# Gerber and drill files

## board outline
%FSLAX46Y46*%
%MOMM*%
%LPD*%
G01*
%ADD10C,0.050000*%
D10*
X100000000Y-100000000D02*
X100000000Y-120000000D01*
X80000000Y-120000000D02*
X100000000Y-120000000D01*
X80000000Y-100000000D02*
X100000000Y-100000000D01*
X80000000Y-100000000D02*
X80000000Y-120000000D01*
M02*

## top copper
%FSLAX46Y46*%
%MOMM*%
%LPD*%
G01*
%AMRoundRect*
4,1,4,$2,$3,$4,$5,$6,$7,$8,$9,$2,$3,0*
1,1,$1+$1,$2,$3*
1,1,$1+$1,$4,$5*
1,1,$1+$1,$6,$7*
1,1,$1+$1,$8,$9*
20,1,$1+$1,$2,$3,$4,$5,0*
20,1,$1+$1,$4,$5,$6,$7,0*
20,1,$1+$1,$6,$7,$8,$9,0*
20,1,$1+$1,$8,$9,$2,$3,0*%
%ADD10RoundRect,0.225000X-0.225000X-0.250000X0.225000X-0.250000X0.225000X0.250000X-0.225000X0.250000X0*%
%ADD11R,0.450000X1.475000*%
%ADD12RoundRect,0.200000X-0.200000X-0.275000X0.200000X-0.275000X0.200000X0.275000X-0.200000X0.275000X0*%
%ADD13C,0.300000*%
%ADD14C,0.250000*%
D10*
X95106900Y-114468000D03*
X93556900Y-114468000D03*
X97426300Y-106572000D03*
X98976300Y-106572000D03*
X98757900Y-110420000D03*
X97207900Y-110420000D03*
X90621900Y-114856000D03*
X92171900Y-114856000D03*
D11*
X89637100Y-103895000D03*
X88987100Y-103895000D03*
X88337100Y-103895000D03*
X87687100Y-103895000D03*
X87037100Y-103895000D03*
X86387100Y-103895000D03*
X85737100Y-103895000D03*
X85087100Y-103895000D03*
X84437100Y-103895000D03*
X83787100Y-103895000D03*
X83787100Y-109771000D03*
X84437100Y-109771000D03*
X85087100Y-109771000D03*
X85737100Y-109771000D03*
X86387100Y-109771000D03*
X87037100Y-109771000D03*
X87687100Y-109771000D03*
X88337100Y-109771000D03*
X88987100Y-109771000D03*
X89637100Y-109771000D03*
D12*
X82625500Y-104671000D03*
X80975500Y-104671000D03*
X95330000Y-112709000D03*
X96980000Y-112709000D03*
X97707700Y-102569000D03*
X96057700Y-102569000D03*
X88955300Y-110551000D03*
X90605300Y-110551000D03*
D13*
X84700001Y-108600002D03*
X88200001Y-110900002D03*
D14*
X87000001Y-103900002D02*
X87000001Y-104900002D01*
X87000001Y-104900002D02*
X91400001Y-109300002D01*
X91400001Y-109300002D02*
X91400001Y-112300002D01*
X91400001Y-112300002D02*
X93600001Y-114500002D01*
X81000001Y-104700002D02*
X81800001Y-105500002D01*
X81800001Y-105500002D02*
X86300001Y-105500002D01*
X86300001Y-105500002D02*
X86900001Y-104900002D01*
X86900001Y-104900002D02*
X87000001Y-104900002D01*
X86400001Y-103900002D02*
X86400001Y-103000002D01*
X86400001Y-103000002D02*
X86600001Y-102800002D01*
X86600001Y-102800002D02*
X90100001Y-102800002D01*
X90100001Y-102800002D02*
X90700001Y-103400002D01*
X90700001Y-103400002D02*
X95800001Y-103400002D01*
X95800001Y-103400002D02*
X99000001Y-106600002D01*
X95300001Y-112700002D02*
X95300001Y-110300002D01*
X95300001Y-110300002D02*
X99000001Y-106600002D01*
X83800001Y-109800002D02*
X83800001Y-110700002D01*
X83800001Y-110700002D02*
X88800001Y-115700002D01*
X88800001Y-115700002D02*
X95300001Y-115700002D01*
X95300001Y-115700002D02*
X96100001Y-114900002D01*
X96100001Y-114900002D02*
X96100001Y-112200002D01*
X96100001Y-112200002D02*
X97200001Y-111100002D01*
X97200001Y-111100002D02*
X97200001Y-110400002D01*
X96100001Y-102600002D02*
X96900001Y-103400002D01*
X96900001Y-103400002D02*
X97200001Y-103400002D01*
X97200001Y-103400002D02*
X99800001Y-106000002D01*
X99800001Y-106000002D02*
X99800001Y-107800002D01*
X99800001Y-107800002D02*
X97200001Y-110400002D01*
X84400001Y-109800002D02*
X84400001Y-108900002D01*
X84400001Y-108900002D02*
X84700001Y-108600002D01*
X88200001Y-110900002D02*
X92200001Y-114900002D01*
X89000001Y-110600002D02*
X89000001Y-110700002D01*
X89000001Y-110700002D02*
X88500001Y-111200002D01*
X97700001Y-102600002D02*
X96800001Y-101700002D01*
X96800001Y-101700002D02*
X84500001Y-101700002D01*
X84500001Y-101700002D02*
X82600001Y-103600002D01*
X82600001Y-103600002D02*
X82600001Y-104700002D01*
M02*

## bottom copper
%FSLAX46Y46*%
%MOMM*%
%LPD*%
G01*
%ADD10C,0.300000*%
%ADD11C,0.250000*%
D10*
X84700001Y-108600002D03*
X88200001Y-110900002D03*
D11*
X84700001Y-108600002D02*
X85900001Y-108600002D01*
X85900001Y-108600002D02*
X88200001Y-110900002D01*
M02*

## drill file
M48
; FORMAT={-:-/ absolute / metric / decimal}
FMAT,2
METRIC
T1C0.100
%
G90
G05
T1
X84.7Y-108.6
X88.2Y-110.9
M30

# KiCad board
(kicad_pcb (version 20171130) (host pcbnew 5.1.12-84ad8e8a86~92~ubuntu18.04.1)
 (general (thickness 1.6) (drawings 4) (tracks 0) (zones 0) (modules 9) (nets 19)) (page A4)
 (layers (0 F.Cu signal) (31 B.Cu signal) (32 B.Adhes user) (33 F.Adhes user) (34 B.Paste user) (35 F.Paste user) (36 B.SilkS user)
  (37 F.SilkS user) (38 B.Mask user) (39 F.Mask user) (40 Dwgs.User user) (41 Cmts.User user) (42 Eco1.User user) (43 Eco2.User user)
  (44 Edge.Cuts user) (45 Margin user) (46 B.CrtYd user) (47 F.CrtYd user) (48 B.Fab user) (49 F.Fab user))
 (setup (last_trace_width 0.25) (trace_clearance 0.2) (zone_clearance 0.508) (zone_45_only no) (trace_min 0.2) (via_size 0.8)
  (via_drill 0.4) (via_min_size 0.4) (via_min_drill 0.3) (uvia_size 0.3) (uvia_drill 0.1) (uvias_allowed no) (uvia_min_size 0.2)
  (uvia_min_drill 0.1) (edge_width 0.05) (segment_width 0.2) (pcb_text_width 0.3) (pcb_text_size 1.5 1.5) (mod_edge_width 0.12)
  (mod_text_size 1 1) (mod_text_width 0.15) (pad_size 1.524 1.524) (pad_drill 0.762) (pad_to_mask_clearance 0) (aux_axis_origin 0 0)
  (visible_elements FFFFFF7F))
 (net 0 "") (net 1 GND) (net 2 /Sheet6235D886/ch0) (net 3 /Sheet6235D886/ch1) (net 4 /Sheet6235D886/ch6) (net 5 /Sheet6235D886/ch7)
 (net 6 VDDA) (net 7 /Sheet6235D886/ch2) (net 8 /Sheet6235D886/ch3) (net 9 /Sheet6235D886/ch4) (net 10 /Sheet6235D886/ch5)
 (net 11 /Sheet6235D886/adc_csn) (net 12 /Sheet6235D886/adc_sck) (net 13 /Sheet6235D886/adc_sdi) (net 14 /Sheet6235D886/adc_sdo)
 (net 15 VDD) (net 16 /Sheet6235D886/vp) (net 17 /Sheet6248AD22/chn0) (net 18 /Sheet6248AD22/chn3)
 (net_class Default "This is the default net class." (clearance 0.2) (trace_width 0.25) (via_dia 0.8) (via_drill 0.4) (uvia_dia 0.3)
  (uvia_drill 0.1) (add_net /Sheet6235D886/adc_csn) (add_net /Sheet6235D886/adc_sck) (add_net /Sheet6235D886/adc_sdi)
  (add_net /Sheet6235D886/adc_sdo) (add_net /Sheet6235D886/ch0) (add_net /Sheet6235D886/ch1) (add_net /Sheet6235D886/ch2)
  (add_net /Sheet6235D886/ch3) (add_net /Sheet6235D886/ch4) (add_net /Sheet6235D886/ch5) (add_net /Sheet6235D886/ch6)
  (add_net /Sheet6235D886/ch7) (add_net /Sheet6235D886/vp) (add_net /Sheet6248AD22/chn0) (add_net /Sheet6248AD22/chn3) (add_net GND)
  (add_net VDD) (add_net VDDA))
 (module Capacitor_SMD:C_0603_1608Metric (layer F.Cu) (at 94.331900 114.468000)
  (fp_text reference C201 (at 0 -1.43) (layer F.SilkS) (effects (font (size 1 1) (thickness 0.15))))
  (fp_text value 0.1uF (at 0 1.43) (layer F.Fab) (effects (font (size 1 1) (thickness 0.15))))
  (pad 2 smd roundrect (at 0.775 0) (size 0.9 0.95) (layers F.Cu F.Mask F.Paste) (roundrect_rratio 0.25) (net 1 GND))
  (pad 1 smd roundrect (at -0.775 0) (size 0.9 0.95) (layers F.Cu F.Mask F.Paste) (roundrect_rratio 0.25) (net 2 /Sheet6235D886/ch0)))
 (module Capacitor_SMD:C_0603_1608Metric (layer F.Cu) (at 98.201300 106.572000)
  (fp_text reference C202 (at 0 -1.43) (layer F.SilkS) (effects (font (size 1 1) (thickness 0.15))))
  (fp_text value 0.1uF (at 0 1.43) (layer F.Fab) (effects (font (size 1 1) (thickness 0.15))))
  (pad 1 smd roundrect (at -0.775 0) (size 0.9 0.95) (layers F.Cu F.Mask F.Paste) (roundrect_rratio 0.25) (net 1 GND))
  (pad 2 smd roundrect (at 0.775 0) (size 0.9 0.95) (layers F.Cu F.Mask F.Paste) (roundrect_rratio 0.25) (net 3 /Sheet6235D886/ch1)))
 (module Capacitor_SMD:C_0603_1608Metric (layer F.Cu) (at 97.982900 110.420000)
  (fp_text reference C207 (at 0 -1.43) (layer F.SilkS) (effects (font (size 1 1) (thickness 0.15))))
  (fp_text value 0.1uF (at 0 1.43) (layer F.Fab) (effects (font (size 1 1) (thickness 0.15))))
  (pad 2 smd roundrect (at 0.775 0) (size 0.9 0.95) (layers F.Cu F.Mask F.Paste) (roundrect_rratio 0.25) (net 1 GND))
  (pad 1 smd roundrect (at -0.775 0) (size 0.9 0.95) (layers F.Cu F.Mask F.Paste) (roundrect_rratio 0.25) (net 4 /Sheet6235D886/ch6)))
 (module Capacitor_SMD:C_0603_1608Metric (layer F.Cu) (at 91.396900 114.856000)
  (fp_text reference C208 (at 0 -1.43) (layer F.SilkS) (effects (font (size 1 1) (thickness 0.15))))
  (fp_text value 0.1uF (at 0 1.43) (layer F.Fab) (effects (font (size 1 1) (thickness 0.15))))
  (pad 1 smd roundrect (at -0.775 0) (size 0.9 0.95) (layers F.Cu F.Mask F.Paste) (roundrect_rratio 0.25) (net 1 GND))
  (pad 2 smd roundrect (at 0.775 0) (size 0.9 0.95) (layers F.Cu F.Mask F.Paste) (roundrect_rratio 0.25) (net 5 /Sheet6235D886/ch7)))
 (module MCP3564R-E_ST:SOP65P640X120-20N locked (layer F.Cu) (at 86.712100 106.833000 270.000000)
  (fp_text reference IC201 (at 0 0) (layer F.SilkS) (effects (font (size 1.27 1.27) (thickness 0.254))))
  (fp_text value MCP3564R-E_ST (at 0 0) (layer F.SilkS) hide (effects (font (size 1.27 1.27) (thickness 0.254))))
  (pad 1 smd rect (at -2.938 -2.925) (size 0.45 1.475) (layers F.Cu F.Mask F.Paste) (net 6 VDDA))
  (pad 2 smd rect (at -2.938 -2.275) (size 0.45 1.475) (layers F.Cu F.Mask F.Paste) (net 1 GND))
  (pad 3 smd rect (at -2.938 -1.625) (size 0.45 1.475) (layers F.Cu F.Mask F.Paste) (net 1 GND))
  (pad 4 smd rect (at -2.938 -0.975) (size 0.45 1.475) (layers F.Cu F.Mask F.Paste))
  (pad 5 smd rect (at -2.938 -0.325) (size 0.45 1.475) (layers F.Cu F.Mask F.Paste) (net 2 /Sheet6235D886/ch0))
  (pad 6 smd rect (at -2.938 0.325) (size 0.45 1.475) (layers F.Cu F.Mask F.Paste) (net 3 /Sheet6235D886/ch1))
  (pad 7 smd rect (at -2.938 0.975) (size 0.45 1.475) (layers F.Cu F.Mask F.Paste) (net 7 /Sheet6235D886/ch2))
  (pad 8 smd rect (at -2.938 1.625) (size 0.45 1.475) (layers F.Cu F.Mask F.Paste) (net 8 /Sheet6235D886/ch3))
  (pad 9 smd rect (at -2.938 2.275) (size 0.45 1.475) (layers F.Cu F.Mask F.Paste) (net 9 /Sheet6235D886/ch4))
  (pad 10 smd rect (at -2.938 2.925) (size 0.45 1.475) (layers F.Cu F.Mask F.Paste) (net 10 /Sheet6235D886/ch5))
  (pad 11 smd rect (at 2.938 2.925) (size 0.45 1.475) (layers F.Cu F.Mask F.Paste) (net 4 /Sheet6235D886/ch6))
  (pad 12 smd rect (at 2.938 2.275) (size 0.45 1.475) (layers F.Cu F.Mask F.Paste) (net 5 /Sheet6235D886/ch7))
  (pad 13 smd rect (at 2.938 1.625) (size 0.45 1.475) (layers F.Cu F.Mask F.Paste) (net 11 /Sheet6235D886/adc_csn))
  (pad 14 smd rect (at 2.938 0.975) (size 0.45 1.475) (layers F.Cu F.Mask F.Paste) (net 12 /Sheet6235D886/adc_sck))
  (pad 15 smd rect (at 2.938 0.325) (size 0.45 1.475) (layers F.Cu F.Mask F.Paste) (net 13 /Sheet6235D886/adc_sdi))
  (pad 16 smd rect (at 2.938 -0.325) (size 0.45 1.475) (layers F.Cu F.Mask F.Paste) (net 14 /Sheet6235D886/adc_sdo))
  (pad 17 smd rect (at 2.938 -0.975) (size 0.45 1.475) (layers F.Cu F.Mask F.Paste))
  (pad 18 smd rect (at 2.938 -1.625) (size 0.45 1.475) (layers F.Cu F.Mask F.Paste))
  (pad 19 smd rect (at 2.938 -2.275) (size 0.45 1.475) (layers F.Cu F.Mask F.Paste) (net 1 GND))
  (pad 20 smd rect (at 2.938 -2.925) (size 0.45 1.475) (layers F.Cu F.Mask F.Paste) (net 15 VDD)))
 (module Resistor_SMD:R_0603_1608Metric (layer F.Cu) (at 81.800500 104.671000)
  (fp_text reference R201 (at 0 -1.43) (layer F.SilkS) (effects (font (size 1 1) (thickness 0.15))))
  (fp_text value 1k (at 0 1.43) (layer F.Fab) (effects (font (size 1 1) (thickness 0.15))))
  (pad 2 smd roundrect (at 0.825 0) (size 0.8 0.95) (layers F.Cu F.Mask F.Paste) (roundrect_rratio 0.25) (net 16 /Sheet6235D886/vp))
  (pad 1 smd roundrect (at -0.825 0) (size 0.8 0.95) (layers F.Cu F.Mask F.Paste) (roundrect_rratio 0.25) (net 2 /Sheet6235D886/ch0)))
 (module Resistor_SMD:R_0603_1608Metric (layer F.Cu) (at 96.155000 112.709000)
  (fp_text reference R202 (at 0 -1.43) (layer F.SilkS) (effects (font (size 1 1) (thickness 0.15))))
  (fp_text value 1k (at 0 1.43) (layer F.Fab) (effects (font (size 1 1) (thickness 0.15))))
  (pad 1 smd roundrect (at -0.825 0) (size 0.8 0.95) (layers F.Cu F.Mask F.Paste) (roundrect_rratio 0.25) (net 3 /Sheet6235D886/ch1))
  (pad 2 smd roundrect (at 0.825 0) (size 0.8 0.95) (layers F.Cu F.Mask F.Paste) (roundrect_rratio 0.25) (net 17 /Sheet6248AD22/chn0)))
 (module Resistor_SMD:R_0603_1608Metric (layer F.Cu) (at 96.882700 102.569000)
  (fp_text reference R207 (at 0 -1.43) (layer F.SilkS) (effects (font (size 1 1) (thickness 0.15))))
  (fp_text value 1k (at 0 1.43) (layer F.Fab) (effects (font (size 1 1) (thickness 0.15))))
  (pad 2 smd roundrect (at 0.825 0) (size 0.8 0.95) (layers F.Cu F.Mask F.Paste) (roundrect_rratio 0.25) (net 16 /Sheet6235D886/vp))
  (pad 1 smd roundrect (at -0.825 0) (size 0.8 0.95) (layers F.Cu F.Mask F.Paste) (roundrect_rratio 0.25) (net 4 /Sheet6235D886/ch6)))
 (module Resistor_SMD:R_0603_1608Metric (layer F.Cu) (at 89.780300 110.551000)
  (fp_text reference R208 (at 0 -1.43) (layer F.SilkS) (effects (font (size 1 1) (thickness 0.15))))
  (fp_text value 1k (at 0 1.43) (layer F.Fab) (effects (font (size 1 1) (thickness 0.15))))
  (pad 1 smd roundrect (at -0.825 0) (size 0.8 0.95) (layers F.Cu F.Mask F.Paste) (roundrect_rratio 0.25) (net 5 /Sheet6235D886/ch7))
  (pad 2 smd roundrect (at 0.825 0) (size 0.8 0.95) (layers F.Cu F.Mask F.Paste) (roundrect_rratio 0.25) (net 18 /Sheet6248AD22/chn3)))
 (gr_line (start 100 100) (end 100 120) (layer Edge.Cuts) (width 0.05))
 (gr_line (start 80 120) (end 100 120) (layer Edge.Cuts) (width 0.05))
 (gr_line (start 80 100) (end 100 100) (layer Edge.Cuts) (width 0.05))
 (gr_line (start 80 100) (end 80 120) (layer Edge.Cuts) (width 0.05))
 (segment (start 87.000001 103.900002) (end 87.000001 104.900002) (width 0.250000) (layer F.Cu) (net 2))
 (segment (start 87.000001 104.900002) (end 91.400001 109.300002) (width 0.250000) (layer F.Cu) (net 2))
 (segment (start 91.400001 109.300002) (end 91.400001 112.300002) (width 0.250000) (layer F.Cu) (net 2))
 (segment (start 91.400001 112.300002) (end 93.600001 114.500002) (width 0.250000) (layer F.Cu) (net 2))
 (segment (start 81.000001 104.700002) (end 81.800001 105.500002) (width 0.250000) (layer F.Cu) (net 2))
 (segment (start 81.800001 105.500002) (end 86.300001 105.500002) (width 0.250000) (layer F.Cu) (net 2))
 (segment (start 86.300001 105.500002) (end 86.900001 104.900002) (width 0.250000) (layer F.Cu) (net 2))
 (segment (start 86.900001 104.900002) (end 87.000001 104.900002) (width 0.250000) (layer F.Cu) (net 2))
 (segment (start 86.400001 103.900002) (end 86.400001 103.000002) (width 0.250000) (layer F.Cu) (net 3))
 (segment (start 86.400001 103.000002) (end 86.600001 102.800002) (width 0.250000) (layer F.Cu) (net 3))
 (segment (start 86.600001 102.800002) (end 90.100001 102.800002) (width 0.250000) (layer F.Cu) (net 3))
 (segment (start 90.100001 102.800002) (end 90.700001 103.400002) (width 0.250000) (layer F.Cu) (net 3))
 (segment (start 90.700001 103.400002) (end 95.800001 103.400002) (width 0.250000) (layer F.Cu) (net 3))
 (segment (start 95.800001 103.400002) (end 99.000001 106.600002) (width 0.250000) (layer F.Cu) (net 3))
 (segment (start 95.300001 112.700002) (end 95.300001 110.300002) (width 0.250000) (layer F.Cu) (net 3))
 (segment (start 95.300001 110.300002) (end 99.000001 106.600002) (width 0.250000) (layer F.Cu) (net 3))
 (segment (start 83.800001 109.800002) (end 83.800001 110.700002) (width 0.250000) (layer F.Cu) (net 4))
 (segment (start 83.800001 110.700002) (end 88.800001 115.700002) (width 0.250000) (layer F.Cu) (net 4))
 (segment (start 88.800001 115.700002) (end 95.300001 115.700002) (width 0.250000) (layer F.Cu) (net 4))
 (segment (start 95.300001 115.700002) (end 96.100001 114.900002) (width 0.250000) (layer F.Cu) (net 4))
 (segment (start 96.100001 114.900002) (end 96.100001 112.200002) (width 0.250000) (layer F.Cu) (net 4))
 (segment (start 96.100001 112.200002) (end 97.200001 111.100002) (width 0.250000) (layer F.Cu) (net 4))
 (segment (start 97.200001 111.100002) (end 97.200001 110.400002) (width 0.250000) (layer F.Cu) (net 4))
 (segment (start 96.100001 102.600002) (end 96.900001 103.400002) (width 0.250000) (layer F.Cu) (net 4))
 (segment (start 96.900001 103.400002) (end 97.200001 103.400002) (width 0.250000) (layer F.Cu) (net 4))
 (segment (start 97.200001 103.400002) (end 99.800001 106.000002) (width 0.250000) (layer F.Cu) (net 4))
 (segment (start 99.800001 106.000002) (end 99.800001 107.800002) (width 0.250000) (layer F.Cu) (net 4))
 (segment (start 99.800001 107.800002) (end 97.200001 110.400002) (width 0.250000) (layer F.Cu) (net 4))
 (segment (start 84.400001 109.800002) (end 84.400001 108.900002) (width 0.250000) (layer F.Cu) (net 5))
 (segment (start 84.400001 108.900002) (end 84.700001 108.600002) (width 0.250000) (layer F.Cu) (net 5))
 (segment (start 84.700001 108.600002) (end 85.900001 108.600002) (width 0.250000) (layer B.Cu) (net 5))
 (segment (start 85.900001 108.600002) (end 88.200001 110.900002) (width 0.250000) (layer B.Cu) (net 5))
 (segment (start 88.200001 110.900002) (end 92.200001 114.900002) (width 0.250000) (layer F.Cu) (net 5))
 (segment (start 89.000001 110.600002) (end 89.000001 110.700002) (width 0.250000) (layer F.Cu) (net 5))
 (segment (start 89.000001 110.700002) (end 88.500001 111.200002) (width 0.250000) (layer F.Cu) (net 5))
 (via micro (at 84.700001 108.600002) (size 0.300000) (drill 0.100000) (layers F.Cu B.Cu) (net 5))
 (via micro (at 88.200001 110.900002) (size 0.300000) (drill 0.100000) (layers F.Cu B.Cu) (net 5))
 (segment (start 97.700001 102.600002) (end 96.800001 101.700002) (width 0.250000) (layer F.Cu) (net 16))
 (segment (start 96.800001 101.700002) (end 84.500001 101.700002) (width 0.250000) (layer F.Cu) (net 16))
 (segment (start 84.500001 101.700002) (end 82.600001 103.600002) (width 0.250000) (layer F.Cu) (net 16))
 (segment (start 82.600001 103.600002) (end 82.600001 104.700002) (width 0.250000) (layer F.Cu) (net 16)))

